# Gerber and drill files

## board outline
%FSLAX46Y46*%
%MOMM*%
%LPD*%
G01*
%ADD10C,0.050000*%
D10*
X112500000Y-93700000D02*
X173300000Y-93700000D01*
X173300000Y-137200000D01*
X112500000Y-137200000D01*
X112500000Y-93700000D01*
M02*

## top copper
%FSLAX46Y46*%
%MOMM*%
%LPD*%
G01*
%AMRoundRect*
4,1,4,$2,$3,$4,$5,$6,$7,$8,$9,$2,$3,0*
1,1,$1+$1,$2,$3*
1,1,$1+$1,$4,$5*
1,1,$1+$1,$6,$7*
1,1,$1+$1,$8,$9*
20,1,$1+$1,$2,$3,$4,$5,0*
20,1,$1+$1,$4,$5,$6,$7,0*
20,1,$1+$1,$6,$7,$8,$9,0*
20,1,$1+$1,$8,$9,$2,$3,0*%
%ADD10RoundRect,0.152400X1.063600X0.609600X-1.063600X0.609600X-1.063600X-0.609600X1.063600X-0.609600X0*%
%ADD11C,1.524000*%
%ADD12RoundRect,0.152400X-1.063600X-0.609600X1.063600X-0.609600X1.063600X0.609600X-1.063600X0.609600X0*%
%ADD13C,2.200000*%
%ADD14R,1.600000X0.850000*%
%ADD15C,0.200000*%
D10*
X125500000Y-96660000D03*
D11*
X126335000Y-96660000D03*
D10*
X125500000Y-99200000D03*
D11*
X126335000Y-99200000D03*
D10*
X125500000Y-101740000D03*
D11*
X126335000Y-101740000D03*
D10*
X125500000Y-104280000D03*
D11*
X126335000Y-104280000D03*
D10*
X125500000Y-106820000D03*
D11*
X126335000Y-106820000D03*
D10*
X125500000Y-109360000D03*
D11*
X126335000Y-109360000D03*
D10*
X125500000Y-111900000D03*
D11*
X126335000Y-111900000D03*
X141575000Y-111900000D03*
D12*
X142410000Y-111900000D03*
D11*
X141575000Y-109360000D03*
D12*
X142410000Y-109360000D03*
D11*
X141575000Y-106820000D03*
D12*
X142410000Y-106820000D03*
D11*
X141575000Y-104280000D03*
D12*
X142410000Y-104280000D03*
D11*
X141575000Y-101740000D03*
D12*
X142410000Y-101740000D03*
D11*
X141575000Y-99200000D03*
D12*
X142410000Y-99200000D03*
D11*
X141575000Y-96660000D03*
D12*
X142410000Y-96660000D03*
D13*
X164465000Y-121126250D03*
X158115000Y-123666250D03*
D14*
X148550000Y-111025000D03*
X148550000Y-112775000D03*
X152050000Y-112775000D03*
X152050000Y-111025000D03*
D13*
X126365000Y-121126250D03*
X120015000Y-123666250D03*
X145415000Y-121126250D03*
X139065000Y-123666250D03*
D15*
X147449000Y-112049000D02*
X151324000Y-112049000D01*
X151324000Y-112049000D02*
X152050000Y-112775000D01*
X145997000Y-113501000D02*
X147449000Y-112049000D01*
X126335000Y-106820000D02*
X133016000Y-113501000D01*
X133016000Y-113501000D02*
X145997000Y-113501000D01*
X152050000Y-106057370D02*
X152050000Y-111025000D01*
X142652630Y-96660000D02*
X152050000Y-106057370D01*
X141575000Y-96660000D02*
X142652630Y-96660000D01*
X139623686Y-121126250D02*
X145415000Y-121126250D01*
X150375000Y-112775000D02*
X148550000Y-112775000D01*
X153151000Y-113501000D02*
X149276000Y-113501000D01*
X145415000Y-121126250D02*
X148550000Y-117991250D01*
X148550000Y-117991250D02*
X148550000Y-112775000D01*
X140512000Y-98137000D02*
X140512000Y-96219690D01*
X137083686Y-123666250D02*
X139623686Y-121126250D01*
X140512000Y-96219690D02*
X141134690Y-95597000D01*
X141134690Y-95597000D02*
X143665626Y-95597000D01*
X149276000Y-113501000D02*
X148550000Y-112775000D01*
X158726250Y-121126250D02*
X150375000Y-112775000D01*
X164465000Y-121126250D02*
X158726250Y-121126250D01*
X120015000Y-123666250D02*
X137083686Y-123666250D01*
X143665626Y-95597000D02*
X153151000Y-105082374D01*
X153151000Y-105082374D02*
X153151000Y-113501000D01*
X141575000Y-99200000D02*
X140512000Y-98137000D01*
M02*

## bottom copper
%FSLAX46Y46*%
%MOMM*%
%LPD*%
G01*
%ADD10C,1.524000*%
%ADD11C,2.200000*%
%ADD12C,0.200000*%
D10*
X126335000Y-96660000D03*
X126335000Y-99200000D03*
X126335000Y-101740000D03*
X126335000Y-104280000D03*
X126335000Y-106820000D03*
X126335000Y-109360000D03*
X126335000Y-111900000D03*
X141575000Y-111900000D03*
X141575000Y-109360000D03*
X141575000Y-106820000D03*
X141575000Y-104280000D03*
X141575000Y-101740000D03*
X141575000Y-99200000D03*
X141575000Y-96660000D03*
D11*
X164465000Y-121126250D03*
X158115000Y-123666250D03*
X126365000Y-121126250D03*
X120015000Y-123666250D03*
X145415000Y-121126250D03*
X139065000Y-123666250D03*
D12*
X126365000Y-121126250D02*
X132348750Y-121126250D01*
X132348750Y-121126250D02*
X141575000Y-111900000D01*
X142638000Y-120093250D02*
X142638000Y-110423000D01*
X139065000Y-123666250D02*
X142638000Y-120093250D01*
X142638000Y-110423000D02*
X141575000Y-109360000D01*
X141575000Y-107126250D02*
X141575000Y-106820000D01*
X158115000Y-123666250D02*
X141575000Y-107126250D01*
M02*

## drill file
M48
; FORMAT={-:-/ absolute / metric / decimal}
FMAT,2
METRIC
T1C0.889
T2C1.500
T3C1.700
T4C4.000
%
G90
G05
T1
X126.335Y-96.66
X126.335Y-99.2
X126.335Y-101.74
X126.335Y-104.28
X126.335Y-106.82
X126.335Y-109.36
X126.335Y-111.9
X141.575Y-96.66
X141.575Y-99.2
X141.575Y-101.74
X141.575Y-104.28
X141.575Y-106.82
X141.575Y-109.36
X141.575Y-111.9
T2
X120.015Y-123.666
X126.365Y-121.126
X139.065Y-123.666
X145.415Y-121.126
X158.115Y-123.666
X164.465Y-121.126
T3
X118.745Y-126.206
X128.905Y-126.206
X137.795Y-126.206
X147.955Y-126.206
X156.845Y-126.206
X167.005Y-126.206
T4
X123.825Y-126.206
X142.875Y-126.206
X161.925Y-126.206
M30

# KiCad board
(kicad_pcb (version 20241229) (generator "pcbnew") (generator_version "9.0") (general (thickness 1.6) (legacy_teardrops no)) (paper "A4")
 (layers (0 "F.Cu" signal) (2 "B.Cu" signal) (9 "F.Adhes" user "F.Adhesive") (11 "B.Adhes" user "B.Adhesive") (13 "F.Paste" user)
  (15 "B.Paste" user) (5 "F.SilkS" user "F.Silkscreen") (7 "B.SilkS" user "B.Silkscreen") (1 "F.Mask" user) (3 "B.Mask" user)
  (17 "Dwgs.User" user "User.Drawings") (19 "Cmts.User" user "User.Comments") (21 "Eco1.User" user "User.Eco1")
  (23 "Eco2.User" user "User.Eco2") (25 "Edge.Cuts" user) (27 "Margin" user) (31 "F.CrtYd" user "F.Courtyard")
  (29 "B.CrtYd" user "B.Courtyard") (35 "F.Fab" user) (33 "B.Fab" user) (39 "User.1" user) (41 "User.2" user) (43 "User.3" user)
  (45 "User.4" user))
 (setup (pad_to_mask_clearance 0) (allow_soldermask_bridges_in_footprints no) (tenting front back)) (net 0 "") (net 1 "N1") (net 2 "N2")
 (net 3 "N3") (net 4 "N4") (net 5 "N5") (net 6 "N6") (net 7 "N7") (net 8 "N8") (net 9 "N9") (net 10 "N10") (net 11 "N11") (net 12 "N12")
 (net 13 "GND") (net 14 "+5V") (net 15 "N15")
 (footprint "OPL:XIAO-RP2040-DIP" (layer "F.Cu") (at 133.955 104.28)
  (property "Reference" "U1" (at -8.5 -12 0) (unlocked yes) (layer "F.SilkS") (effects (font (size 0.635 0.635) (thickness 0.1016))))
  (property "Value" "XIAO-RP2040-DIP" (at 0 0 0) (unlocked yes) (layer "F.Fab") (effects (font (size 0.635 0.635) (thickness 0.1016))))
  (pad "1" smd roundrect (at -8.455 -7.62 180) (size 2.432 1.524) (layers "F.Cu" "F.Mask") (roundrect_rratio 0.1) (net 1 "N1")
   (thermal_bridge_angle 45))
  (pad "1" thru_hole circle (at -7.62 -7.62 180) (size 1.524 1.524) (drill 0.889) (layers "*.Cu" "*.Mask") (remove_unused_layers no)
   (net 1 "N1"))
  (pad "2" smd roundrect (at -8.455 -5.08 180) (size 2.432 1.524) (layers "F.Cu" "F.Mask") (roundrect_rratio 0.1) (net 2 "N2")
   (thermal_bridge_angle 45))
  (pad "2" thru_hole circle (at -7.62 -5.08 180) (size 1.524 1.524) (drill 0.889) (layers "*.Cu" "*.Mask") (remove_unused_layers no)
   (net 2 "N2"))
  (pad "3" smd roundrect (at -8.455 -2.54 180) (size 2.432 1.524) (layers "F.Cu" "F.Mask") (roundrect_rratio 0.1) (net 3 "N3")
   (thermal_bridge_angle 45))
  (pad "3" thru_hole circle (at -7.62 -2.54 180) (size 1.524 1.524) (drill 0.889) (layers "*.Cu" "*.Mask") (remove_unused_layers no)
   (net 3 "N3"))
  (pad "4" smd roundrect (at -8.455 0 180) (size 2.432 1.524) (layers "F.Cu" "F.Mask") (roundrect_rratio 0.1) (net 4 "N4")
   (thermal_bridge_angle 45))
  (pad "4" thru_hole circle (at -7.62 0 180) (size 1.524 1.524) (drill 0.889) (layers "*.Cu" "*.Mask") (remove_unused_layers no)
   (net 4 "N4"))
  (pad "5" smd roundrect (at -8.455 2.54 180) (size 2.432 1.524) (layers "F.Cu" "F.Mask") (roundrect_rratio 0.1) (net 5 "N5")
   (thermal_bridge_angle 45))
  (pad "5" thru_hole circle (at -7.62 2.54 180) (size 1.524 1.524) (drill 0.889) (layers "*.Cu" "*.Mask") (remove_unused_layers no)
   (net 5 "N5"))
  (pad "6" smd roundrect (at -8.455 5.08 180) (size 2.432 1.524) (layers "F.Cu" "F.Mask") (roundrect_rratio 0.1) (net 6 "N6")
   (thermal_bridge_angle 45))
  (pad "6" thru_hole circle (at -7.62 5.08 180) (size 1.524 1.524) (drill 0.889) (layers "*.Cu" "*.Mask") (remove_unused_layers no)
   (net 6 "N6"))
  (pad "7" smd roundrect (at -8.455 7.62 180) (size 2.432 1.524) (layers "F.Cu" "F.Mask") (roundrect_rratio 0.1) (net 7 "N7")
   (thermal_bridge_angle 45))
  (pad "7" thru_hole circle (at -7.62 7.62 180) (size 1.524 1.524) (drill 0.889) (layers "*.Cu" "*.Mask") (remove_unused_layers no)
   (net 7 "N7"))
  (pad "8" thru_hole circle (at 7.62 7.62) (size 1.524 1.524) (drill 0.889) (layers "*.Cu" "*.Mask") (remove_unused_layers no) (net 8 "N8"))
  (pad "8" smd roundrect (at 8.455 7.62) (size 2.432 1.524) (layers "F.Cu" "F.Mask") (roundrect_rratio 0.1) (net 8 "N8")
   (thermal_bridge_angle 45))
  (pad "9" thru_hole circle (at 7.62 5.08) (size 1.524 1.524) (drill 0.889) (layers "*.Cu" "*.Mask") (remove_unused_layers no) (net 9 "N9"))
  (pad "9" smd roundrect (at 8.455 5.08) (size 2.432 1.524) (layers "F.Cu" "F.Mask") (roundrect_rratio 0.1) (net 9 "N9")
   (thermal_bridge_angle 45))
  (pad "10" thru_hole circle (at 7.62 2.54) (size 1.524 1.524) (drill 0.889) (layers "*.Cu" "*.Mask") (remove_unused_layers no)
   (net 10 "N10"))
  (pad "10" smd roundrect (at 8.455 2.54) (size 2.432 1.524) (layers "F.Cu" "F.Mask") (roundrect_rratio 0.1) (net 10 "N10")
   (thermal_bridge_angle 45))
  (pad "11" thru_hole circle (at 7.62 0) (size 1.524 1.524) (drill 0.889) (layers "*.Cu" "*.Mask") (remove_unused_layers no) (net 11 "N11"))
  (pad "11" smd roundrect (at 8.455 0) (size 2.432 1.524) (layers "F.Cu" "F.Mask") (roundrect_rratio 0.1) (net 11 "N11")
   (thermal_bridge_angle 45))
  (pad "12" thru_hole circle (at 7.62 -2.54) (size 1.524 1.524) (drill 0.889) (layers "*.Cu" "*.Mask") (remove_unused_layers no)
   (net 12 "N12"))
  (pad "12" smd roundrect (at 8.455 -2.54) (size 2.432 1.524) (layers "F.Cu" "F.Mask") (roundrect_rratio 0.1) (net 12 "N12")
   (thermal_bridge_angle 45))
  (pad "13" thru_hole circle (at 7.62 -5.08) (size 1.524 1.524) (drill 0.889) (layers "*.Cu" "*.Mask") (remove_unused_layers no)
   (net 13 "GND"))
  (pad "13" smd roundrect (at 8.455 -5.08) (size 2.432 1.524) (layers "F.Cu" "F.Mask") (roundrect_rratio 0.1) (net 13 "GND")
   (thermal_bridge_angle 45))
  (pad "14" thru_hole circle (at 7.62 -7.62) (size 1.524 1.524) (drill 0.889) (layers "*.Cu" "*.Mask") (remove_unused_layers no)
   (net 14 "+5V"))
  (pad "14" smd roundrect (at 8.455 -7.62) (size 2.432 1.524) (layers "F.Cu" "F.Mask") (roundrect_rratio 0.1) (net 14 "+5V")
   (thermal_bridge_angle 45)))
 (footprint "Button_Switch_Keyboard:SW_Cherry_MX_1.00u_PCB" (layer "F.Cu") (at 164.465 121.12625)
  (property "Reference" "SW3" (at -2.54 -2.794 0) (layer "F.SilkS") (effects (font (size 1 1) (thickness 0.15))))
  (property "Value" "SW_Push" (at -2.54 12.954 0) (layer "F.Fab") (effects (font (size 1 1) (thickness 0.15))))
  (pad "" np_thru_hole circle (at -7.62 5.08) (size 1.7 1.7) (drill 1.7) (layers "*.Cu" "*.Mask"))
  (pad "" np_thru_hole circle (at -2.54 5.08) (size 4 4) (drill 4) (layers "*.Cu" "*.Mask"))
  (pad "" np_thru_hole circle (at 2.54 5.08) (size 1.7 1.7) (drill 1.7) (layers "*.Cu" "*.Mask"))
  (pad "1" thru_hole circle (at 0 0) (size 2.2 2.2) (drill 1.5) (layers "*.Cu" "*.Mask") (remove_unused_layers no) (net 13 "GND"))
  (pad "2" thru_hole circle (at -6.35 2.54) (size 2.2 2.2) (drill 1.5) (layers "*.Cu" "*.Mask") (remove_unused_layers no) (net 10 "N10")))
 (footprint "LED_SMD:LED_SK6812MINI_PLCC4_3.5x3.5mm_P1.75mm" (layer "F.Cu") (at 150.3 111.9)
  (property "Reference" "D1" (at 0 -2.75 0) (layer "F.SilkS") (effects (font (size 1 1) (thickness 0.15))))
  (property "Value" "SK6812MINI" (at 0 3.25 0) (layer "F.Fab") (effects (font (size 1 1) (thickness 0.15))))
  (pad "1" smd rect (at -1.75 -0.875) (size 1.6 0.85) (layers "F.Cu" "F.Mask" "F.Paste") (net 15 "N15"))
  (pad "2" smd rect (at -1.75 0.875) (size 1.6 0.85) (layers "F.Cu" "F.Mask" "F.Paste") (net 13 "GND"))
  (pad "3" smd rect (at 1.75 0.875) (size 1.6 0.85) (layers "F.Cu" "F.Mask" "F.Paste") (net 5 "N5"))
  (pad "4" smd rect (at 1.75 -0.875) (size 1.6 0.85) (layers "F.Cu" "F.Mask" "F.Paste") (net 14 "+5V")))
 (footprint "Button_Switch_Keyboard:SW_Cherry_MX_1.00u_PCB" (layer "F.Cu") (at 126.365 121.12625)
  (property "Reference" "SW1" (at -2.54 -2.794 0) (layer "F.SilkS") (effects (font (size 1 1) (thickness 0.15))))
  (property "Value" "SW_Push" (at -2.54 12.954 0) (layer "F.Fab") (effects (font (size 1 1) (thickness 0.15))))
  (pad "" np_thru_hole circle (at -7.62 5.08) (size 1.7 1.7) (drill 1.7) (layers "*.Cu" "*.Mask"))
  (pad "" np_thru_hole circle (at -2.54 5.08) (size 4 4) (drill 4) (layers "*.Cu" "*.Mask"))
  (pad "" np_thru_hole circle (at 2.54 5.08) (size 1.7 1.7) (drill 1.7) (layers "*.Cu" "*.Mask"))
  (pad "1" thru_hole circle (at 0 0) (size 2.2 2.2) (drill 1.5) (layers "*.Cu" "*.Mask") (remove_unused_layers no) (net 8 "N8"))
  (pad "2" thru_hole circle (at -6.35 2.54) (size 2.2 2.2) (drill 1.5) (layers "*.Cu" "*.Mask") (remove_unused_layers no) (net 13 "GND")))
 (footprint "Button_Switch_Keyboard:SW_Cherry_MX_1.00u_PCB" (layer "F.Cu") (at 145.415 121.12625)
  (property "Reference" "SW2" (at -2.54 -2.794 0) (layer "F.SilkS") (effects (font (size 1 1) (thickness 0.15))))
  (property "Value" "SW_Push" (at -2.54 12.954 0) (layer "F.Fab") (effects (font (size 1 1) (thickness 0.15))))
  (pad "" np_thru_hole circle (at -7.62 5.08) (size 1.7 1.7) (drill 1.7) (layers "*.Cu" "*.Mask"))
  (pad "" np_thru_hole circle (at -2.54 5.08) (size 4 4) (drill 4) (layers "*.Cu" "*.Mask"))
  (pad "" np_thru_hole circle (at 2.54 5.08) (size 1.7 1.7) (drill 1.7) (layers "*.Cu" "*.Mask"))
  (pad "1" thru_hole circle (at 0 0) (size 2.2 2.2) (drill 1.5) (layers "*.Cu" "*.Mask") (remove_unused_layers no) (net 13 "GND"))
  (pad "2" thru_hole circle (at -6.35 2.54) (size 2.2 2.2) (drill 1.5) (layers "*.Cu" "*.Mask") (remove_unused_layers no) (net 9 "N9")))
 (gr_rect (start 112.5 93.7) (end 173.3 137.2) (stroke (width 0.05) (type default)) (fill no) (layer "Edge.Cuts"))
 (segment (start 147.449 112.049) (end 151.324 112.049) (width 0.2) (layer "F.Cu") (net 5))
 (segment (start 151.324 112.049) (end 152.05 112.775) (width 0.2) (layer "F.Cu") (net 5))
 (segment (start 145.997 113.501) (end 147.449 112.049) (width 0.2) (layer "F.Cu") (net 5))
 (segment (start 126.335 106.82) (end 133.016 113.501) (width 0.2) (layer "F.Cu") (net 5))
 (segment (start 133.016 113.501) (end 145.997 113.501) (width 0.2) (layer "F.Cu") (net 5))
 (segment (start 152.05 106.05737) (end 152.05 111.025) (width 0.2) (layer "F.Cu") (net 14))
 (segment (start 142.65263 96.66) (end 152.05 106.05737) (width 0.2) (layer "F.Cu") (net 14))
 (segment (start 141.575 96.66) (end 142.65263 96.66) (width 0.2) (layer "F.Cu") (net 14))
 (segment (start 139.623686 121.12625) (end 145.415 121.12625) (width 0.2) (layer "F.Cu") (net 13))
 (segment (start 150.375 112.775) (end 148.55 112.775) (width 0.2) (layer "F.Cu") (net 13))
 (segment (start 153.151 113.501) (end 149.276 113.501) (width 0.2) (layer "F.Cu") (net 13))
 (segment (start 145.415 121.12625) (end 148.55 117.99125) (width 0.2) (layer "F.Cu") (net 13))
 (segment (start 148.55 117.99125) (end 148.55 112.775) (width 0.2) (layer "F.Cu") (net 13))
 (segment (start 140.512 98.137) (end 140.512 96.21969) (width 0.2) (layer "F.Cu") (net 13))
 (segment (start 137.083686 123.66625) (end 139.623686 121.12625) (width 0.2) (layer "F.Cu") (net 13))
 (segment (start 140.512 96.21969) (end 141.13469 95.597) (width 0.2) (layer "F.Cu") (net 13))
 (segment (start 141.13469 95.597) (end 143.665626 95.597) (width 0.2) (layer "F.Cu") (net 13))
 (segment (start 149.276 113.501) (end 148.55 112.775) (width 0.2) (layer "F.Cu") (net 13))
 (segment (start 158.72625 121.12625) (end 150.375 112.775) (width 0.2) (layer "F.Cu") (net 13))
 (segment (start 164.465 121.12625) (end 158.72625 121.12625) (width 0.2) (layer "F.Cu") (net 13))
 (segment (start 120.015 123.66625) (end 137.083686 123.66625) (width 0.2) (layer "F.Cu") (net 13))
 (segment (start 143.665626 95.597) (end 153.151 105.082374) (width 0.2) (layer "F.Cu") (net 13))
 (segment (start 153.151 105.082374) (end 153.151 113.501) (width 0.2) (layer "F.Cu") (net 13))
 (segment (start 141.575 99.2) (end 140.512 98.137) (width 0.2) (layer "F.Cu") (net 13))
 (segment (start 126.365 121.12625) (end 132.34875 121.12625) (width 0.2) (layer "B.Cu") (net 8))
 (segment (start 132.34875 121.12625) (end 141.575 111.9) (width 0.2) (layer "B.Cu") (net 8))
 (segment (start 142.638 120.09325) (end 142.638 110.423) (width 0.2) (layer "B.Cu") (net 9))
 (segment (start 139.065 123.66625) (end 142.638 120.09325) (width 0.2) (layer "B.Cu") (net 9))
 (segment (start 142.638 110.423) (end 141.575 109.36) (width 0.2) (layer "B.Cu") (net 9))
 (segment (start 141.575 107.12625) (end 141.575 106.82) (width 0.2) (layer "B.Cu") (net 10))
 (segment (start 158.115 123.66625) (end 141.575 107.12625) (width 0.2) (layer "B.Cu") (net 10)))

